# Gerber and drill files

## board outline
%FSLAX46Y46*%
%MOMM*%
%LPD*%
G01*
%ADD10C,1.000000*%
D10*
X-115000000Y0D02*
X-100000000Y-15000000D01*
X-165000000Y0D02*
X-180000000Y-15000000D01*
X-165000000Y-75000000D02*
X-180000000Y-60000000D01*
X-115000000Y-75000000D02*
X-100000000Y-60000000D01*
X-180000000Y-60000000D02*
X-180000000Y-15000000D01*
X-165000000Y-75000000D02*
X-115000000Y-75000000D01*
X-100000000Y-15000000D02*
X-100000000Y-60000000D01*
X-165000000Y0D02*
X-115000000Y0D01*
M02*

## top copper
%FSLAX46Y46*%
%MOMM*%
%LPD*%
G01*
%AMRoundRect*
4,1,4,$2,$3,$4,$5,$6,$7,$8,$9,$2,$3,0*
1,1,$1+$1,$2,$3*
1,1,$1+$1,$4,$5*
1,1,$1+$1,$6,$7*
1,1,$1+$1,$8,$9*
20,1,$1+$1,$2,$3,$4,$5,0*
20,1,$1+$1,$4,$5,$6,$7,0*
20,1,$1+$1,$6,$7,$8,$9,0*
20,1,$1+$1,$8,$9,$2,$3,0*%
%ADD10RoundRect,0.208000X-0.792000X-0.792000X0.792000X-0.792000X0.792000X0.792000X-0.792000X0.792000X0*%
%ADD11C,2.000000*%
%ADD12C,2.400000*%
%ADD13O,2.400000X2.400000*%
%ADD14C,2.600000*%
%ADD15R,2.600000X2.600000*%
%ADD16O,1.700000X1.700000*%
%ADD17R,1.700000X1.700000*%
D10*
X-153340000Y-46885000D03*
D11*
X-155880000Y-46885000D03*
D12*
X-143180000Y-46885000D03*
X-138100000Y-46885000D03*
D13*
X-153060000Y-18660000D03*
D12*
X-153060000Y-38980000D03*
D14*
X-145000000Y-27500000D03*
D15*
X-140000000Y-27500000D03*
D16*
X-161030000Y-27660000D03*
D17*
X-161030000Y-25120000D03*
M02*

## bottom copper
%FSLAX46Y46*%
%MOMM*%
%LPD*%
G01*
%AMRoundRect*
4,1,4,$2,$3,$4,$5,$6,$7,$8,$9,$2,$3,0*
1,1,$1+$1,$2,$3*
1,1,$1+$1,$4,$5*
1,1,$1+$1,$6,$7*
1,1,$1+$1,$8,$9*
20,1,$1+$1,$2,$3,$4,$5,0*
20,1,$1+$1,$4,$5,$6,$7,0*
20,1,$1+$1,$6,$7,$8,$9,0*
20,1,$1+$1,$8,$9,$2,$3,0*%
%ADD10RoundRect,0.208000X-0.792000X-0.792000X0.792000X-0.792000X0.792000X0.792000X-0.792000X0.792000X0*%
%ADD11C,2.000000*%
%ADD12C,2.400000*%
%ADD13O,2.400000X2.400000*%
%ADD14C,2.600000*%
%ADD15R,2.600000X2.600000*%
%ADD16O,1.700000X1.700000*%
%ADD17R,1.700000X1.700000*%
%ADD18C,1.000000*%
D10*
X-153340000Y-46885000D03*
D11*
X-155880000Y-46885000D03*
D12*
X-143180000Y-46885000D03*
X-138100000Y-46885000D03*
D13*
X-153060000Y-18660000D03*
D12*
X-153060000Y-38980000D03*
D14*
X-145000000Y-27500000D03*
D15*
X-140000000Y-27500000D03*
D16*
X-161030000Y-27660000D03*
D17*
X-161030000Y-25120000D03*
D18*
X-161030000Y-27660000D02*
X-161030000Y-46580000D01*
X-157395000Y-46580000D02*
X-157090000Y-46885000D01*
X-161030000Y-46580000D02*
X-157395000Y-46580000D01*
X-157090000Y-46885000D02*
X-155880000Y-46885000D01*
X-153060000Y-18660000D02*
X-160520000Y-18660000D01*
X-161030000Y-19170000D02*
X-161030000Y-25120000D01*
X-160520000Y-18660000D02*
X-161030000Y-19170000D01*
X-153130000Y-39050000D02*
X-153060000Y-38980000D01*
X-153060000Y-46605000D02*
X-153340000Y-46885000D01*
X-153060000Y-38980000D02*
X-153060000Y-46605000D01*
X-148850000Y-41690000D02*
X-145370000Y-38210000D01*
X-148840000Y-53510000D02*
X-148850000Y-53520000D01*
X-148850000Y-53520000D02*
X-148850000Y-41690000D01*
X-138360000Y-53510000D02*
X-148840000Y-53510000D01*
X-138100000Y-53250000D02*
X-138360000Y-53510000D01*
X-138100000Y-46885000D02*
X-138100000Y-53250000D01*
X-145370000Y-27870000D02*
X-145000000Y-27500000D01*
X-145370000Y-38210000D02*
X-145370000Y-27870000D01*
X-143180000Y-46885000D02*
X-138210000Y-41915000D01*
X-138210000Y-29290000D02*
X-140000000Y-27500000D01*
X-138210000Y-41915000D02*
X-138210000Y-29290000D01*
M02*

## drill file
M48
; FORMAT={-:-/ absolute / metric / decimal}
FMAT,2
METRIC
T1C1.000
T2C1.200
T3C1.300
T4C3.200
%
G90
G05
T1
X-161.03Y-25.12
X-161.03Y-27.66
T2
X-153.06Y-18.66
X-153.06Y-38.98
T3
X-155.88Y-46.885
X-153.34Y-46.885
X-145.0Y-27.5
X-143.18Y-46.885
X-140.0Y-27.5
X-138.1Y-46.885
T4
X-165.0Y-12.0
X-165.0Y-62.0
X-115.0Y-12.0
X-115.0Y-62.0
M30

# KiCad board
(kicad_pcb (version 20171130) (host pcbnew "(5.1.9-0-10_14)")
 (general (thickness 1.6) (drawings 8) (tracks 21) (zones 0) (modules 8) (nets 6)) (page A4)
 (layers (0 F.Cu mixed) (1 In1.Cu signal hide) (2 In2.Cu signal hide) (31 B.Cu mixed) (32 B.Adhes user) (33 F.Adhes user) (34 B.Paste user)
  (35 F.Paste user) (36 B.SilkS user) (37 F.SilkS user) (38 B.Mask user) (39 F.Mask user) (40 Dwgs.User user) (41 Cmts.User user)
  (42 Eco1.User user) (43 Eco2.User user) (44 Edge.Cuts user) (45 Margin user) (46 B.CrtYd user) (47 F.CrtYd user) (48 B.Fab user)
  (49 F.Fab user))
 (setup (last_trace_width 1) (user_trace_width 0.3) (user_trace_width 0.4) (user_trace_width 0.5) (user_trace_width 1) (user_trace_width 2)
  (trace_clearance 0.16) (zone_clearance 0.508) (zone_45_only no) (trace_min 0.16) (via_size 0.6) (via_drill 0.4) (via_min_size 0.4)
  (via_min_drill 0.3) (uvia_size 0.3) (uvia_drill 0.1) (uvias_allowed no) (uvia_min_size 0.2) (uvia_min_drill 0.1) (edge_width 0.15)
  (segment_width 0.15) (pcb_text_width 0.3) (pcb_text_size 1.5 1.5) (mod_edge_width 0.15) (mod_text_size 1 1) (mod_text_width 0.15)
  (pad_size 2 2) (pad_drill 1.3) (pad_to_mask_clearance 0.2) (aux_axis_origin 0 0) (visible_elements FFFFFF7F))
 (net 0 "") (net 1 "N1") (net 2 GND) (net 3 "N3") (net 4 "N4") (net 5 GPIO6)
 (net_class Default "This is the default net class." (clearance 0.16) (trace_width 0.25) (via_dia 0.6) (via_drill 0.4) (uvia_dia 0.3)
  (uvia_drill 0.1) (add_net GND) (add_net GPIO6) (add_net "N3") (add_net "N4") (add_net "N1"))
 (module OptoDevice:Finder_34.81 (layer F.Cu) (at -153.34 46.885)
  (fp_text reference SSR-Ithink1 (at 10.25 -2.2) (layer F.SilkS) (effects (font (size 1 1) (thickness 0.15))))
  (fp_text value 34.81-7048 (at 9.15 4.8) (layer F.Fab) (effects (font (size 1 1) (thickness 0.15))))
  (pad A1 thru_hole roundrect (at 0 0) (size 2 2) (drill 1.3) (layers *.Cu *.Mask) (roundrect_rratio 0.104) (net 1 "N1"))
  (pad A2 thru_hole circle (at -2.54 0) (size 2 2) (drill 1.3) (layers *.Cu *.Mask) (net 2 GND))
  (pad 11 thru_hole circle (at 10.16 0) (size 2.4 2.4) (drill 1.3) (layers *.Cu *.Mask) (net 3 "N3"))
  (pad 14 thru_hole circle (at 15.24 0) (size 2.4 2.4) (drill 1.3) (layers *.Cu *.Mask) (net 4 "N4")))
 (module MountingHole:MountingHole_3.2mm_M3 (layer F.Cu) (at -165 62)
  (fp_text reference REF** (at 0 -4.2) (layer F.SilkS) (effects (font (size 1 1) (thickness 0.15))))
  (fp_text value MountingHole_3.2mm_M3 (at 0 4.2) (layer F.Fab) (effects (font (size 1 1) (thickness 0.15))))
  (pad 1 np_thru_hole circle (at 0 0) (size 3.2 3.2) (drill 3.2) (layers *.Cu *.Mask)))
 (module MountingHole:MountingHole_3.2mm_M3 (layer F.Cu) (at -115 62)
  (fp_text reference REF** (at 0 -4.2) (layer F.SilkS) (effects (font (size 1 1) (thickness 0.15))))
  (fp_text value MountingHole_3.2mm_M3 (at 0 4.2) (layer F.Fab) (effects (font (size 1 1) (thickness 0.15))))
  (pad 1 np_thru_hole circle (at 0 0) (size 3.2 3.2) (drill 3.2) (layers *.Cu *.Mask)))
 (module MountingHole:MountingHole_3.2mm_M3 (layer F.Cu) (at -115 12)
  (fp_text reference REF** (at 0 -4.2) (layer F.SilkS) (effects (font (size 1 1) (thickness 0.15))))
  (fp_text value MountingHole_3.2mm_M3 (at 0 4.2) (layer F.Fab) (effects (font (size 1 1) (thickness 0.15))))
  (pad 1 np_thru_hole circle (at 0 0) (size 3.2 3.2) (drill 3.2) (layers *.Cu *.Mask)))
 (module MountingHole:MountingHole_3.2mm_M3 (layer F.Cu) (at -165 12)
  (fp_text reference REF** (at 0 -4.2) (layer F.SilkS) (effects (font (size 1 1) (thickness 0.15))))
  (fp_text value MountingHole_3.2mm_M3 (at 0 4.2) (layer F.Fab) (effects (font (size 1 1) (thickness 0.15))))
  (pad 1 np_thru_hole circle (at 0 0) (size 3.2 3.2) (drill 3.2) (layers *.Cu *.Mask)))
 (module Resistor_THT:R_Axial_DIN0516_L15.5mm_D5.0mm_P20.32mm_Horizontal (layer F.Cu) (at -153.06 38.98 90)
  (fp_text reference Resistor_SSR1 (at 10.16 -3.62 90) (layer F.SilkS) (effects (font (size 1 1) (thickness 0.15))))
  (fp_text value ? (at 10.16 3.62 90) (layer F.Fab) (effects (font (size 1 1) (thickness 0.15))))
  (pad 2 thru_hole oval (at 20.32 0 90) (size 2.4 2.4) (drill 1.2) (layers *.Cu *.Mask) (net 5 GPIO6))
  (pad 1 thru_hole circle (at 0 0 90) (size 2.4 2.4) (drill 1.2) (layers *.Cu *.Mask) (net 1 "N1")))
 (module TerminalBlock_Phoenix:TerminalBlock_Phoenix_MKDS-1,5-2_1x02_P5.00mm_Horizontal (layer F.Cu) (at -140 27.5 180)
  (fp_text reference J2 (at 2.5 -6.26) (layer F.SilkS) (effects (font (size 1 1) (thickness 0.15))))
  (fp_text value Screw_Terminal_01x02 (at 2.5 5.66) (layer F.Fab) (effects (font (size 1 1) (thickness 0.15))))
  (pad 2 thru_hole circle (at 5 0 180) (size 2.6 2.6) (drill 1.3) (layers *.Cu *.Mask) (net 4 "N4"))
  (pad 1 thru_hole rect (at 0 0 180) (size 2.6 2.6) (drill 1.3) (layers *.Cu *.Mask) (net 3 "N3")))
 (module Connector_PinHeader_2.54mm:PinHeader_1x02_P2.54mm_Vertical (layer F.Cu) (at -161.03 25.12)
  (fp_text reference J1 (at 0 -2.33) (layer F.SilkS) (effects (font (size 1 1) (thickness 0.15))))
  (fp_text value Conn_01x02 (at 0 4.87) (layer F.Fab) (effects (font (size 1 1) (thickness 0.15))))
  (pad 2 thru_hole oval (at 0 2.54) (size 1.7 1.7) (drill 1) (layers *.Cu *.Mask) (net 2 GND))
  (pad 1 thru_hole rect (at 0 0) (size 1.7 1.7) (drill 1) (layers *.Cu *.Mask) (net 5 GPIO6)))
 (gr_line (start -115 0) (end -100 15) (layer Edge.Cuts) (width 1))
 (gr_line (start -165 0) (end -180 15) (layer Edge.Cuts) (width 1))
 (gr_line (start -165 75) (end -180 60) (layer Edge.Cuts) (width 1))
 (gr_line (start -115 75) (end -100 60) (layer Edge.Cuts) (width 1))
 (gr_line (start -180 60) (end -180 15) (layer Edge.Cuts) (width 1))
 (gr_line (start -165 75) (end -115 75) (layer Edge.Cuts) (width 1))
 (gr_line (start -100 15) (end -100 60) (layer Edge.Cuts) (width 1))
 (gr_line (start -165 0) (end -115 0) (layer Edge.Cuts) (width 1))
 (segment (start -161.03 27.66) (end -161.03 46.58) (width 1) (layer B.Cu) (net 2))
 (segment (start -157.395 46.58) (end -157.09 46.885) (width 1) (layer B.Cu) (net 2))
 (segment (start -161.03 46.58) (end -157.395 46.58) (width 1) (layer B.Cu) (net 2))
 (segment (start -157.09 46.885) (end -155.88 46.885) (width 1) (layer B.Cu) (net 2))
 (segment (start -153.06 18.66) (end -160.52 18.66) (width 1) (layer B.Cu) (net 5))
 (segment (start -161.03 19.17) (end -161.03 25.12) (width 1) (layer B.Cu) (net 5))
 (segment (start -160.52 18.66) (end -161.03 19.17) (width 1) (layer B.Cu) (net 5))
 (segment (start -153.13 39.05) (end -153.06 38.98) (width 1) (layer B.Cu) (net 1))
 (segment (start -153.06 46.605) (end -153.34 46.885) (width 1) (layer B.Cu) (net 1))
 (segment (start -153.06 38.98) (end -153.06 46.605) (width 1) (layer B.Cu) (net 1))
 (segment (start -148.85 41.69) (end -145.37 38.21) (width 1) (layer B.Cu) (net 4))
 (segment (start -148.84 53.51) (end -148.85 53.52) (width 1) (layer B.Cu) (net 4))
 (segment (start -148.85 53.52) (end -148.85 41.69) (width 1) (layer B.Cu) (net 4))
 (segment (start -138.36 53.51) (end -148.84 53.51) (width 1) (layer B.Cu) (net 4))
 (segment (start -138.1 53.25) (end -138.36 53.51) (width 1) (layer B.Cu) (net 4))
 (segment (start -138.1 46.885) (end -138.1 53.25) (width 1) (layer B.Cu) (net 4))
 (segment (start -145.37 27.87) (end -145 27.5) (width 1) (layer B.Cu) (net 4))
 (segment (start -145.37 38.21) (end -145.37 27.87) (width 1) (layer B.Cu) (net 4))
 (segment (start -143.18 46.885) (end -138.21 41.915) (width 1) (layer B.Cu) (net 3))
 (segment (start -138.21 29.29) (end -140 27.5) (width 1) (layer B.Cu) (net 3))
 (segment (start -138.21 41.915) (end -138.21 29.29) (width 1) (layer B.Cu) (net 3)))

